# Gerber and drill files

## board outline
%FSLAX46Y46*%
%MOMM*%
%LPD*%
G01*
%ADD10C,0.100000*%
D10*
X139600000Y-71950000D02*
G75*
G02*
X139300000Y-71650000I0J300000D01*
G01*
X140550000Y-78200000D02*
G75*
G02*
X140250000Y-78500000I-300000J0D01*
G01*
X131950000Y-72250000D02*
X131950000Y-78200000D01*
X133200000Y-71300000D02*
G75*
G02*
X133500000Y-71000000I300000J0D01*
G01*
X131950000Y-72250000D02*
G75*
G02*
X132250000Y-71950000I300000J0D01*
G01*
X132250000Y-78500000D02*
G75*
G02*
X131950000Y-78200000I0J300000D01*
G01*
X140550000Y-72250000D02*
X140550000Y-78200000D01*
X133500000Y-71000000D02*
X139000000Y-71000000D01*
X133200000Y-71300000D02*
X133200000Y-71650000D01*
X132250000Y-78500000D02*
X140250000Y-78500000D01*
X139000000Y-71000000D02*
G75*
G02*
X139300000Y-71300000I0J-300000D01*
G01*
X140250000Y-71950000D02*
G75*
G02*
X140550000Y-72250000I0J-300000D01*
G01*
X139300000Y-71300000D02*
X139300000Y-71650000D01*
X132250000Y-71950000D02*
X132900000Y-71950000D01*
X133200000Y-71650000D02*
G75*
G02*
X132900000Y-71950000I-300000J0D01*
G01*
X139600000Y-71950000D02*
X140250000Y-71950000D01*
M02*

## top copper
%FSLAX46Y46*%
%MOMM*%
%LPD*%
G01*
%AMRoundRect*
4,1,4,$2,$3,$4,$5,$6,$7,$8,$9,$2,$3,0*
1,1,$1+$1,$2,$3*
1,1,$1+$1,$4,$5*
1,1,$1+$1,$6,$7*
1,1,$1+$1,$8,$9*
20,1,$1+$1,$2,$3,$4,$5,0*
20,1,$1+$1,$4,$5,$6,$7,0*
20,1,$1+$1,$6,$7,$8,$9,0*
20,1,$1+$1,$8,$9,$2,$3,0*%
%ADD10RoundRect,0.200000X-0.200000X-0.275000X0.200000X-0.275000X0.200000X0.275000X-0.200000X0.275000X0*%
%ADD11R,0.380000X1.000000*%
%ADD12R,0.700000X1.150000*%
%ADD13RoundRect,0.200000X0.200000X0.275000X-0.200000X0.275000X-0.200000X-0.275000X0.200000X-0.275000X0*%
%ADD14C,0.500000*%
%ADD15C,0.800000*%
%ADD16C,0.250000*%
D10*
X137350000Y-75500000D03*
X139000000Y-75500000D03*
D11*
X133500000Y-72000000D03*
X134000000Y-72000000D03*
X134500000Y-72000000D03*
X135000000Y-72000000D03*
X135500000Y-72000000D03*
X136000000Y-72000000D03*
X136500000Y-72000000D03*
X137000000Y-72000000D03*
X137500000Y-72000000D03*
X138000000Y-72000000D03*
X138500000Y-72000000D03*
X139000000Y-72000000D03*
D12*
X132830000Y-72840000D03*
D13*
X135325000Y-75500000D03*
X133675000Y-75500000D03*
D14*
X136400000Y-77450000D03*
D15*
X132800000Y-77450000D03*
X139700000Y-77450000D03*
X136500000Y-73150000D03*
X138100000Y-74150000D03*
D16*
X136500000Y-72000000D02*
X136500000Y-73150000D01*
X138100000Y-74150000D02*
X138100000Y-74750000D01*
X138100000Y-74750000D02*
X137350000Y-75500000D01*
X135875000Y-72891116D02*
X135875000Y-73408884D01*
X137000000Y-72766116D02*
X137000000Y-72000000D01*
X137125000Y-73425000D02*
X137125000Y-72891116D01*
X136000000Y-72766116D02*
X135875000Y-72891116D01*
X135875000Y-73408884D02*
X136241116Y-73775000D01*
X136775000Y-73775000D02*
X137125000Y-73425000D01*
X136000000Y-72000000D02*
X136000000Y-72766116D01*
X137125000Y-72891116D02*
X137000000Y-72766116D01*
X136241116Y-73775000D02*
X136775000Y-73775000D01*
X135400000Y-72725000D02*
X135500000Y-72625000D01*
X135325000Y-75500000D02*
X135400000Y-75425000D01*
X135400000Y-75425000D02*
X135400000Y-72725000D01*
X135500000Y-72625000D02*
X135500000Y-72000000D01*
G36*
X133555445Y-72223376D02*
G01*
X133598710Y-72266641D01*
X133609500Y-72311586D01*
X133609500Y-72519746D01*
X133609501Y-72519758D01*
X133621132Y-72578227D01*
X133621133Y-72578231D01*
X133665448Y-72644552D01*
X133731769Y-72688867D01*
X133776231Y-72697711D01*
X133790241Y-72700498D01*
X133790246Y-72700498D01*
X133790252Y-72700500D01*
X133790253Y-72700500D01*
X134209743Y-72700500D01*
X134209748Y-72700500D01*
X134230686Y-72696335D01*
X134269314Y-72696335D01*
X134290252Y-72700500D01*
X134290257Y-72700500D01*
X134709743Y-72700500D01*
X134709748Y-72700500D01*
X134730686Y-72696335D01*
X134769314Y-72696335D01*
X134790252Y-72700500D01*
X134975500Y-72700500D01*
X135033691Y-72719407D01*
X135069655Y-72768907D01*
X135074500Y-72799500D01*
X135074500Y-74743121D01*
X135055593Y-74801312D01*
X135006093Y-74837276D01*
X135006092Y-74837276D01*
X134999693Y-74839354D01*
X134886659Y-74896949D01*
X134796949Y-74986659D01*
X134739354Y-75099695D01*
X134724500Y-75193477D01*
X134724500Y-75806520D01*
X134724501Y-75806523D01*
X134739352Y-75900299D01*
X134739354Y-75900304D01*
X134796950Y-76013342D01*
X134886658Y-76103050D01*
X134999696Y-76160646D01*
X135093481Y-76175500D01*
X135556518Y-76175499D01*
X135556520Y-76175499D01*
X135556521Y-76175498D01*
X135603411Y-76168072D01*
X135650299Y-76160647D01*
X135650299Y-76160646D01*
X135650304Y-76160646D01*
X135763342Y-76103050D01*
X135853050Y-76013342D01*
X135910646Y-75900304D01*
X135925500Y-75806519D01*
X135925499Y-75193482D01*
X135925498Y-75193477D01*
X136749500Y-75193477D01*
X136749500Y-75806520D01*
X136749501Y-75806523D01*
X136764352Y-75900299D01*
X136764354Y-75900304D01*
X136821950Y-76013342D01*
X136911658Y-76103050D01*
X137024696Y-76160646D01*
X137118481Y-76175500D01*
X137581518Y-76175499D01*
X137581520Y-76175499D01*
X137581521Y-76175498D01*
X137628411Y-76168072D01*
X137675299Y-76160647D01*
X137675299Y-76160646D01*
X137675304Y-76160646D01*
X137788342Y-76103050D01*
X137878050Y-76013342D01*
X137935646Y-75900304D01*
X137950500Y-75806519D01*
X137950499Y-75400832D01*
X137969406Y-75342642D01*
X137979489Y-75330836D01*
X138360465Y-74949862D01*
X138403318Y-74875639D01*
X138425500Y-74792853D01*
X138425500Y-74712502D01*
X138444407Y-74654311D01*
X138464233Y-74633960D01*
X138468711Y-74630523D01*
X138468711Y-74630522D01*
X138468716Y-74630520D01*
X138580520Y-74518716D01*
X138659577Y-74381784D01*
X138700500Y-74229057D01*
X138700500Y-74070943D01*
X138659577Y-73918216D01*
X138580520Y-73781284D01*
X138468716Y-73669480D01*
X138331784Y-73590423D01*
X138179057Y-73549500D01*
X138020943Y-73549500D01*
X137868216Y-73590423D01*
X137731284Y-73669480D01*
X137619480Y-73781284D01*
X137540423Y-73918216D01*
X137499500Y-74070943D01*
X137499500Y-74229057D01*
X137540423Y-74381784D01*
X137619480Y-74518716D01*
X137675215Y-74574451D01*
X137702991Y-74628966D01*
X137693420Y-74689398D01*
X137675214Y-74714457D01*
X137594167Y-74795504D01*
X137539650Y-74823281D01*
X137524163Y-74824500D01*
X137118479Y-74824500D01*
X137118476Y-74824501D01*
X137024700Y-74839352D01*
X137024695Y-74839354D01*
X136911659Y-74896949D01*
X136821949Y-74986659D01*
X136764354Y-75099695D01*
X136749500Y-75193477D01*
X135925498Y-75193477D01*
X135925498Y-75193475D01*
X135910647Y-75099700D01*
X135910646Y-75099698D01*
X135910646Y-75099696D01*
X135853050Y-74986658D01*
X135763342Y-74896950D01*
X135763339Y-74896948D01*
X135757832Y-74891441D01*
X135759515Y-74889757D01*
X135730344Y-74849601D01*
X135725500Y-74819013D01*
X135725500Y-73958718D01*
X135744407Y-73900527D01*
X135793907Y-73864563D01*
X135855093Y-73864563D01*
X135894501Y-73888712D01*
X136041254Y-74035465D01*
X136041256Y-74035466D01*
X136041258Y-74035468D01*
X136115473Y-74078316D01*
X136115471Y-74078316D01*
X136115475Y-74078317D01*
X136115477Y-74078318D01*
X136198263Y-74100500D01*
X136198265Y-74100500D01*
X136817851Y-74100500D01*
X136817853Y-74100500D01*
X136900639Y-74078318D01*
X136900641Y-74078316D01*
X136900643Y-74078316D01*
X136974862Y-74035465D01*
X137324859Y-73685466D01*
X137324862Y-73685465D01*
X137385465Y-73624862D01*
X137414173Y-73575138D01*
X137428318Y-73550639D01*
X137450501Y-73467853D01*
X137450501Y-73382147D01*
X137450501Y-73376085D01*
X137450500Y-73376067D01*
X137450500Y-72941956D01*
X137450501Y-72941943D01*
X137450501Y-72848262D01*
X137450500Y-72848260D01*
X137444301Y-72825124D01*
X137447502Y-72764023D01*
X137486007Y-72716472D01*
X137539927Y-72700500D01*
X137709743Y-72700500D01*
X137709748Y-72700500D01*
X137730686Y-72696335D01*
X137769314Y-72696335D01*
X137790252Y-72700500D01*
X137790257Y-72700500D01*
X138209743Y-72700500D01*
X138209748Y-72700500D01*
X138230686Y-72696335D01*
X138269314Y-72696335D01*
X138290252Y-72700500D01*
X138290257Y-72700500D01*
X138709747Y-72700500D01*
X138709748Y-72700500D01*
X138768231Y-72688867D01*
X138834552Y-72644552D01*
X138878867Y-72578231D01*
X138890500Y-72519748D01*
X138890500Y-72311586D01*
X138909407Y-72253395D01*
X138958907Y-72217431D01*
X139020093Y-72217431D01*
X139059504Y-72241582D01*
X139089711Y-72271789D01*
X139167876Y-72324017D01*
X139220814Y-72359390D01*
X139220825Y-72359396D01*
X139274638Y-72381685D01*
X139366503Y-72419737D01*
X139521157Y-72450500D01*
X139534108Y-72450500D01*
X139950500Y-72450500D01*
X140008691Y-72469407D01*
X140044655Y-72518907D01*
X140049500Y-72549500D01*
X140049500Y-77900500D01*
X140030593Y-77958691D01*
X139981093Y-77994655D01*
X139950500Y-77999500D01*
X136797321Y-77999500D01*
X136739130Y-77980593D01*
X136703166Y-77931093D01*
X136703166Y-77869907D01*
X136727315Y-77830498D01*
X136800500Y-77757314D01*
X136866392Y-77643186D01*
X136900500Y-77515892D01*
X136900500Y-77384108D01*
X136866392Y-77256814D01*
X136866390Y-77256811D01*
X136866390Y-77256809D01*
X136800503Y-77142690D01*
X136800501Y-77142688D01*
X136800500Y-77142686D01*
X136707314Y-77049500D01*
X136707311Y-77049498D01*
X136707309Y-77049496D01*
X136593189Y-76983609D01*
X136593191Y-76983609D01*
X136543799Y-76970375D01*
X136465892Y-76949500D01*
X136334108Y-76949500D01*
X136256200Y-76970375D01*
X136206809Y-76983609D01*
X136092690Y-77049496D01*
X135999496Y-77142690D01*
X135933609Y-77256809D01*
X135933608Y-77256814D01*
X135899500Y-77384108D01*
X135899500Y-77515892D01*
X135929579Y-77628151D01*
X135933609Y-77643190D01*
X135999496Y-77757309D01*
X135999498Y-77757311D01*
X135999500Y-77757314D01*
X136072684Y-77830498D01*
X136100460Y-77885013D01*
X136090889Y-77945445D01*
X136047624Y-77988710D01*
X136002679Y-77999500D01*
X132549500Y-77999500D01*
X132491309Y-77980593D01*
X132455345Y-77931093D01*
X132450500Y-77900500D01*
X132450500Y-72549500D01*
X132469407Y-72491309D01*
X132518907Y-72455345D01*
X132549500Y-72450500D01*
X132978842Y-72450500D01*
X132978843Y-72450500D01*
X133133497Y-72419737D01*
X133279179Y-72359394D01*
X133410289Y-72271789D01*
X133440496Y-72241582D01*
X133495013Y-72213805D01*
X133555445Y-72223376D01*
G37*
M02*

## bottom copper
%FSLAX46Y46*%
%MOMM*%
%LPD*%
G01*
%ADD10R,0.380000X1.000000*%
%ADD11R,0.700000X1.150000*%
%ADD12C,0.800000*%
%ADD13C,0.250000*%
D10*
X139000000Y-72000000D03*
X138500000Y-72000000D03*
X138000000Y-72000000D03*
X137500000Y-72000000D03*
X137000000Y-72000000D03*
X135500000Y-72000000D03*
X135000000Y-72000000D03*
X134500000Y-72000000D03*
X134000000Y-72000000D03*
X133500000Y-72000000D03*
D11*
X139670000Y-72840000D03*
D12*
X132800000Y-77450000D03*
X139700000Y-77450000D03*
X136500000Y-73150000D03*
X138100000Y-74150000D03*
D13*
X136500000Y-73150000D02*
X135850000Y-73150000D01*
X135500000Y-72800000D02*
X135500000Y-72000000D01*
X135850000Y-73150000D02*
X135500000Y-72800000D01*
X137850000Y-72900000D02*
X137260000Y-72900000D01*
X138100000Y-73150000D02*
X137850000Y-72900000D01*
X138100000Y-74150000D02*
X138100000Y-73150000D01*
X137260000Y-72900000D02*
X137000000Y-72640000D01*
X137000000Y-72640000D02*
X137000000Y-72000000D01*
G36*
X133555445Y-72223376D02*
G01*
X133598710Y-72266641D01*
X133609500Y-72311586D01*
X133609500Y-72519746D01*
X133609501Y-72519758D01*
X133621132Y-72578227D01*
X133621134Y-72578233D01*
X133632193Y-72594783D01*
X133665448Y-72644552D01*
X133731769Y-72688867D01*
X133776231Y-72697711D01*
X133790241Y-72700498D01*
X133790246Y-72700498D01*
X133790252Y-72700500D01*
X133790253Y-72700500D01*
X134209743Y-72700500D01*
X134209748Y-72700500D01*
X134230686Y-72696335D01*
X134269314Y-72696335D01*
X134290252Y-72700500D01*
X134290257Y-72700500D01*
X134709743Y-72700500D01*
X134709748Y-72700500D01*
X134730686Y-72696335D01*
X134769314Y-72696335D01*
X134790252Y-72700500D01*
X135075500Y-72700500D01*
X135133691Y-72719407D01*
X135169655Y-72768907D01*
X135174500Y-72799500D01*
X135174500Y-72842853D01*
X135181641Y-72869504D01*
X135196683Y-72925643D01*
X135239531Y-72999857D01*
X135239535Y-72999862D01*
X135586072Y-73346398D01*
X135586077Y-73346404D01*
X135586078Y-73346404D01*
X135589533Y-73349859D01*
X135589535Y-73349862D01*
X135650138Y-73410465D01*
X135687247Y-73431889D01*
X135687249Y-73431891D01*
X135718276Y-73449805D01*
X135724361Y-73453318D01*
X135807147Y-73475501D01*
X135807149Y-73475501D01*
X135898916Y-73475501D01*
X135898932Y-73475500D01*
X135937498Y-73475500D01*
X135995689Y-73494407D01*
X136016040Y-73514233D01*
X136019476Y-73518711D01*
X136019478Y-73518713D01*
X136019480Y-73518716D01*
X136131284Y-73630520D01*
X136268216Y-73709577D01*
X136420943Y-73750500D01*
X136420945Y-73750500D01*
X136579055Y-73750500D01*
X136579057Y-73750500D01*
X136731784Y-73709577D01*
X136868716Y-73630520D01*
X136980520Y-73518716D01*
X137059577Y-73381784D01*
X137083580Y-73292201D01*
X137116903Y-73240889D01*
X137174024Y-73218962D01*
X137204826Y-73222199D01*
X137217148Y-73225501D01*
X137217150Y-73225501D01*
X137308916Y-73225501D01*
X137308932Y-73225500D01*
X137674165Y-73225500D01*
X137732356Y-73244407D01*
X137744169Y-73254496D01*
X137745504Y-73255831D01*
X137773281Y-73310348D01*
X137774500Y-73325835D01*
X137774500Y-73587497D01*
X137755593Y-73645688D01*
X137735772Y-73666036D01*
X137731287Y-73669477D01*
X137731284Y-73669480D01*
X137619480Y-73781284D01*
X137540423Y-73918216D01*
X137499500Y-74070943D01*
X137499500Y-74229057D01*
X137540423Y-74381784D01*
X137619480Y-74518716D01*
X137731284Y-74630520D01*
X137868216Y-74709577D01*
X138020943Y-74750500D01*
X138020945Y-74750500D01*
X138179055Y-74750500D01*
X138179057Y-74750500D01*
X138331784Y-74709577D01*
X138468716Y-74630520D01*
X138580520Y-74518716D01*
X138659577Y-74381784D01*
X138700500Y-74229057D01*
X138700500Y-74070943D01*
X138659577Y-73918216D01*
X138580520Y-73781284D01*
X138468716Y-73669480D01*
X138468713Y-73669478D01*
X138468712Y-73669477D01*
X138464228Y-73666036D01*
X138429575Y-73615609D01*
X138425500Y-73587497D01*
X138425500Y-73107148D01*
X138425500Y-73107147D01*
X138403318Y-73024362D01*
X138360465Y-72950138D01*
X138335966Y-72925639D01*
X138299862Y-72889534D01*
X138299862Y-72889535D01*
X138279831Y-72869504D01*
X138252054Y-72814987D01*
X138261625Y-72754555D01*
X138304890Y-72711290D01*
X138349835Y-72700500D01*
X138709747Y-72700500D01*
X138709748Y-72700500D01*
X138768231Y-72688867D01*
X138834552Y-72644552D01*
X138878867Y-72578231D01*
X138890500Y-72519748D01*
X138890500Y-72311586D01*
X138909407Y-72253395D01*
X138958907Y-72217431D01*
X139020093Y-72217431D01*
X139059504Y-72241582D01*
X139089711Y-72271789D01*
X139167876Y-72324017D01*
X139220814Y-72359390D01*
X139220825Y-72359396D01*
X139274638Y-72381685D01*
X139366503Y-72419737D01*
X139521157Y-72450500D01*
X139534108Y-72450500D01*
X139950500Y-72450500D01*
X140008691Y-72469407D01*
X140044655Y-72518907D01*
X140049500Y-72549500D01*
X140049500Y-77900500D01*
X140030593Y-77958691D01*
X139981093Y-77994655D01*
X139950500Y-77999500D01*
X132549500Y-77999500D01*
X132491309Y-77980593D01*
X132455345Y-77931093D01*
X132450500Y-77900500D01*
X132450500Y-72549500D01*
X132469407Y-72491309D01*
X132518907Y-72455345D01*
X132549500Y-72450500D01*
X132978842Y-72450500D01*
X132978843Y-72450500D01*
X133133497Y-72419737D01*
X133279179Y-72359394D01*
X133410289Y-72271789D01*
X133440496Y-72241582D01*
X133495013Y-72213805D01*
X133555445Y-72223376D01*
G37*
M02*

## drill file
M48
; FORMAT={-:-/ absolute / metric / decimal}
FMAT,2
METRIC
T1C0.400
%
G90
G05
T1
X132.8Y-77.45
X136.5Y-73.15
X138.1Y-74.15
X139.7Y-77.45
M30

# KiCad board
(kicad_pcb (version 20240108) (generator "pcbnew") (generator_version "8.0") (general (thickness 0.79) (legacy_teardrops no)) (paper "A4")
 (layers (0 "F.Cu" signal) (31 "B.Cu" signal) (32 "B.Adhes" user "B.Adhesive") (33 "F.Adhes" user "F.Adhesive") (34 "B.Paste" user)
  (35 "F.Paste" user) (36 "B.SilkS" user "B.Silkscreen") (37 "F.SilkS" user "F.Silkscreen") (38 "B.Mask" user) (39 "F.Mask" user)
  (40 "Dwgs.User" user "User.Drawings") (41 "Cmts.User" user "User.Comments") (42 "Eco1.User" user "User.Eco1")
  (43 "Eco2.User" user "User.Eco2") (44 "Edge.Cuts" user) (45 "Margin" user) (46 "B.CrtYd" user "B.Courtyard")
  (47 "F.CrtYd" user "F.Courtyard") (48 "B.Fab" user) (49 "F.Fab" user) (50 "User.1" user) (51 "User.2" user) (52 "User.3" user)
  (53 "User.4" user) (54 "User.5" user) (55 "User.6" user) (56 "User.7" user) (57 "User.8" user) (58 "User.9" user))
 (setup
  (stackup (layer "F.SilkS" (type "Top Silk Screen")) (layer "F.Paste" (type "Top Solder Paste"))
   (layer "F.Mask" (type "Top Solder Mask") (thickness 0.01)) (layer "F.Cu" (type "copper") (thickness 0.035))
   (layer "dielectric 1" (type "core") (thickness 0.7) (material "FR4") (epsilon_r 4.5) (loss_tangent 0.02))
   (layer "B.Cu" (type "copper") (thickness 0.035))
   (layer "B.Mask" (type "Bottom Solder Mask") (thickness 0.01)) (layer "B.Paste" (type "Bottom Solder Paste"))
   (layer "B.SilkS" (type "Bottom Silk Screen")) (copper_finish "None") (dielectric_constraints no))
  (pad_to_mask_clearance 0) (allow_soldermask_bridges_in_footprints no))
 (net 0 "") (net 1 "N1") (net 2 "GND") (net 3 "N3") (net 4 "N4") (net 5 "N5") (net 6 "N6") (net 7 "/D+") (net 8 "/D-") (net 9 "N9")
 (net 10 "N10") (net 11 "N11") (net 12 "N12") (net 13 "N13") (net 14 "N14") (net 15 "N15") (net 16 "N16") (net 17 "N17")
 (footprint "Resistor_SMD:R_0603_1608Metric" (layer "F.Cu") (at 138.175 75.5)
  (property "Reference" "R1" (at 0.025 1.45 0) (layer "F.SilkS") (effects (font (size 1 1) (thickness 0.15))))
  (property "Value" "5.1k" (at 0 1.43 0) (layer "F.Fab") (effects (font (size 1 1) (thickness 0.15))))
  (pad "1" smd roundrect (at -0.825 0) (size 0.8 0.95) (layers "F.Cu" "F.Paste" "F.Mask") (roundrect_rratio 0.25) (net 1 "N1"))
  (pad "2" smd roundrect (at 0.825 0) (size 0.8 0.95) (layers "F.Cu" "F.Paste" "F.Mask") (roundrect_rratio 0.25) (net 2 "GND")))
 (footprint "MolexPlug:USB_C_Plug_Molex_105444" (layer "F.Cu") (at 136.25 71.96)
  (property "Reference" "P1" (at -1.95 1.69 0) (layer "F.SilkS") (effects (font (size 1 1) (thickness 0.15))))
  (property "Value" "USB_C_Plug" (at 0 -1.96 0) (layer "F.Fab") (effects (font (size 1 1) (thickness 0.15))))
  (pad "A1" smd rect (at -2.75 0.04) (size 0.38 1) (layers "F.Cu" "F.Paste" "F.Mask") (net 2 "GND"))
  (pad "A2" smd rect (at -2.25 0.04) (size 0.38 1) (layers "F.Cu" "F.Paste" "F.Mask") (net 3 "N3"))
  (pad "A3" smd rect (at -1.75 0.04) (size 0.38 1) (layers "F.Cu" "F.Paste" "F.Mask") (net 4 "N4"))
  (pad "A4" smd rect (at -1.25 0.04) (size 0.38 1) (layers "F.Cu" "F.Paste" "F.Mask") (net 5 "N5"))
  (pad "A5" smd rect (at -0.75 0.04) (size 0.38 1) (layers "F.Cu" "F.Paste" "F.Mask") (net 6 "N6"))
  (pad "A6" smd rect (at -0.25 0.04) (size 0.38 1) (layers "F.Cu" "F.Paste" "F.Mask") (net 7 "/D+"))
  (pad "A7" smd rect (at 0.25 0.04) (size 0.38 1) (layers "F.Cu" "F.Paste" "F.Mask") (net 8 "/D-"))
  (pad "A8" smd rect (at 0.75 0.04) (size 0.38 1) (layers "F.Cu" "F.Paste" "F.Mask") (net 7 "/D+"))
  (pad "A9" smd rect (at 1.25 0.04) (size 0.38 1) (layers "F.Cu" "F.Paste" "F.Mask") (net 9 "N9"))
  (pad "A10" smd rect (at 1.75 0.04) (size 0.38 1) (layers "F.Cu" "F.Paste" "F.Mask") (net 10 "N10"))
  (pad "A11" smd rect (at 2.25 0.04) (size 0.38 1) (layers "F.Cu" "F.Paste" "F.Mask") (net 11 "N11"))
  (pad "A12" smd rect (at 2.75 0.04) (size 0.38 1) (layers "F.Cu" "F.Paste" "F.Mask") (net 2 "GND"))
  (pad "B1" smd rect (at 2.75 0.04) (size 0.38 1) (layers "B.Cu" "B.Paste" "B.Mask") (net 2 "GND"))
  (pad "B2" smd rect (at 2.25 0.04) (size 0.38 1) (layers "B.Cu" "B.Paste" "B.Mask") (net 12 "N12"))
  (pad "B3" smd rect (at 1.75 0.04) (size 0.38 1) (layers "B.Cu" "B.Paste" "B.Mask") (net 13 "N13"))
  (pad "B4" smd rect (at 1.25 0.04) (size 0.38 1) (layers "B.Cu" "B.Paste" "B.Mask") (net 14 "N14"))
  (pad "B5" smd rect (at 0.75 0.04) (size 0.38 1) (layers "B.Cu" "B.Paste" "B.Mask") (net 1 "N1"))
  (pad "B8" smd rect (at -0.75 0.04) (size 0.38 1) (layers "B.Cu" "B.Paste" "B.Mask") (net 8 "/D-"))
  (pad "B9" smd rect (at -1.25 0.04) (size 0.38 1) (layers "B.Cu" "B.Paste" "B.Mask") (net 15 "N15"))
  (pad "B10" smd rect (at -1.75 0.04) (size 0.38 1) (layers "B.Cu" "B.Paste" "B.Mask") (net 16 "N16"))
  (pad "B11" smd rect (at -2.25 0.04) (size 0.38 1) (layers "B.Cu" "B.Paste" "B.Mask") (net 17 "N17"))
  (pad "B12" smd rect (at -2.75 0.04) (size 0.38 1) (layers "B.Cu" "B.Paste" "B.Mask") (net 2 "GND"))
  (pad "S1" smd rect (at -3.42 0.88) (size 0.7 1.15) (layers "F.Cu" "F.Paste" "F.Mask") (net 2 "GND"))
  (pad "S1" smd rect (at 3.42 0.88) (size 0.7 1.15) (layers "B.Cu" "B.Paste" "B.Mask") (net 2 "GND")))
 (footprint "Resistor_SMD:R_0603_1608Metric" (layer "F.Cu") (at 134.5 75.5 180)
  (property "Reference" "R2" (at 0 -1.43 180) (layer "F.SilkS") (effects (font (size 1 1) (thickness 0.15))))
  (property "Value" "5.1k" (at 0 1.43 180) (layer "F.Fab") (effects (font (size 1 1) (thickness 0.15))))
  (pad "1" smd roundrect (at -0.825 0 180) (size 0.8 0.95) (layers "F.Cu" "F.Paste" "F.Mask") (roundrect_rratio 0.25) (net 6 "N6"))
  (pad "2" smd roundrect (at 0.825 0 180) (size 0.8 0.95) (layers "F.Cu" "F.Paste" "F.Mask") (roundrect_rratio 0.25) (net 2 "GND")))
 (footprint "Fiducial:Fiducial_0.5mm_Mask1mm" (layer "F.Cu") (at 136.4 77.45)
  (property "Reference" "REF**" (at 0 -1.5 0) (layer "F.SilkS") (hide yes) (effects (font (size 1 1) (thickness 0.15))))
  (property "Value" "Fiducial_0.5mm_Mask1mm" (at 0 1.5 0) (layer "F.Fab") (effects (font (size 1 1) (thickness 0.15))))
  (pad "" smd circle (at 0 0) (size 0.5 0.5) (layers "F.Cu" "F.Mask") (solder_mask_margin 0.25) (clearance 0.25)))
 (gr_arc (start 139.6 71.95) (mid 139.387868 71.862132) (end 139.3 71.65) (stroke (width 0.1) (type default)) (layer "Edge.Cuts"))
 (gr_arc (start 140.55 78.2) (mid 140.462132 78.412132) (end 140.25 78.5) (stroke (width 0.1) (type default)) (layer "Edge.Cuts"))
 (gr_line (start 131.95 72.25) (end 131.95 78.2) (stroke (width 0.1) (type default)) (layer "Edge.Cuts"))
 (gr_arc (start 133.2 71.3) (mid 133.287868 71.087868) (end 133.5 71) (stroke (width 0.1) (type default)) (layer "Edge.Cuts"))
 (gr_arc (start 131.95 72.25) (mid 132.037868 72.037868) (end 132.25 71.95) (stroke (width 0.1) (type default)) (layer "Edge.Cuts"))
 (gr_arc (start 132.25 78.5) (mid 132.037868 78.412132) (end 131.95 78.2) (stroke (width 0.1) (type default)) (layer "Edge.Cuts"))
 (gr_line (start 140.55 72.25) (end 140.55 78.2) (stroke (width 0.1) (type default)) (layer "Edge.Cuts"))
 (gr_line (start 133.5 71) (end 139 71) (stroke (width 0.1) (type default)) (layer "Edge.Cuts"))
 (gr_line (start 133.2 71.3) (end 133.2 71.65) (stroke (width 0.1) (type default)) (layer "Edge.Cuts"))
 (gr_line (start 132.25 78.5) (end 140.25 78.5) (stroke (width 0.1) (type default)) (layer "Edge.Cuts"))
 (gr_arc (start 139 71) (mid 139.212132 71.087868) (end 139.3 71.3) (stroke (width 0.1) (type default)) (layer "Edge.Cuts"))
 (gr_arc (start 140.25 71.95) (mid 140.462132 72.037868) (end 140.55 72.25) (stroke (width 0.1) (type default)) (layer "Edge.Cuts"))
 (gr_line (start 139.3 71.3) (end 139.3 71.65) (stroke (width 0.1) (type default)) (layer "Edge.Cuts"))
 (gr_line (start 132.25 71.95) (end 132.9 71.95) (stroke (width 0.1) (type default)) (layer "Edge.Cuts"))
 (gr_arc (start 133.2 71.65) (mid 133.112132 71.862132) (end 132.9 71.95) (stroke (width 0.1) (type default)) (layer "Edge.Cuts"))
 (gr_line (start 139.6 71.95) (end 140.25 71.95) (stroke (width 0.1) (type default)) (layer "Edge.Cuts"))
 (via (at 132.8 77.45) (size 0.8) (drill 0.4) (layers "F.Cu" "B.Cu") (free yes) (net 2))
 (via (at 139.7 77.45) (size 0.8) (drill 0.4) (layers "F.Cu" "B.Cu") (free yes) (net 2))
 (segment (start 136.5 72) (end 136.5 73.15) (width 0.25) (layer "F.Cu") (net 8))
 (via (at 136.5 73.15) (size 0.8) (drill 0.4) (layers "F.Cu" "B.Cu") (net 8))
 (segment (start 136.5 73.15) (end 135.85 73.15) (width 0.25) (layer "B.Cu") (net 8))
 (segment (start 135.5 72.8) (end 135.5 72) (width 0.25) (layer "B.Cu") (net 8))
 (segment (start 135.85 73.15) (end 135.5 72.8) (width 0.25) (layer "B.Cu") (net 8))
 (segment (start 138.1 74.15) (end 138.1 74.75) (width 0.25) (layer "F.Cu") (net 1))
 (segment (start 138.1 74.75) (end 137.35 75.5) (width 0.25) (layer "F.Cu") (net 1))
 (via (at 138.1 74.15) (size 0.8) (drill 0.4) (layers "F.Cu" "B.Cu") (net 1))
 (segment (start 137.85 72.9) (end 137.26 72.9) (width 0.25) (layer "B.Cu") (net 1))
 (segment (start 138.1 73.15) (end 137.85 72.9) (width 0.25) (layer "B.Cu") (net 1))
 (segment (start 138.1 74.15) (end 138.1 73.15) (width 0.25) (layer "B.Cu") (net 1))
 (segment (start 137.26 72.9) (end 137 72.64) (width 0.25) (layer "B.Cu") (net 1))
 (segment (start 137 72.64) (end 137 72) (width 0.25) (layer "B.Cu") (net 1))
 (segment (start 135.875 72.891116) (end 135.875 73.408884) (width 0.25) (layer "F.Cu") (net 7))
 (segment (start 137 72.766116) (end 137 72) (width 0.25) (layer "F.Cu") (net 7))
 (segment (start 137.125 73.425) (end 137.125 72.891116) (width 0.25) (layer "F.Cu") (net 7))
 (segment (start 136 72.766116) (end 135.875 72.891116) (width 0.25) (layer "F.Cu") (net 7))
 (segment (start 135.875 73.408884) (end 136.241116 73.775) (width 0.25) (layer "F.Cu") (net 7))
 (segment (start 136.775 73.775) (end 137.125 73.425) (width 0.25) (layer "F.Cu") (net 7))
 (segment (start 136 72) (end 136 72.766116) (width 0.25) (layer "F.Cu") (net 7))
 (segment (start 137.125 72.891116) (end 137 72.766116) (width 0.25) (layer "F.Cu") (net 7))
 (segment (start 136.241116 73.775) (end 136.775 73.775) (width 0.25) (layer "F.Cu") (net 7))
 (segment (start 135.4 72.725) (end 135.5 72.625) (width 0.25) (layer "F.Cu") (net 6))
 (segment (start 135.325 75.5) (end 135.4 75.425) (width 0.25) (layer "F.Cu") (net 6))
 (segment (start 135.4 75.425) (end 135.4 72.725) (width 0.25) (layer "F.Cu") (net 6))
 (segment (start 135.5 72.625) (end 135.5 72) (width 0.25) (layer "F.Cu") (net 6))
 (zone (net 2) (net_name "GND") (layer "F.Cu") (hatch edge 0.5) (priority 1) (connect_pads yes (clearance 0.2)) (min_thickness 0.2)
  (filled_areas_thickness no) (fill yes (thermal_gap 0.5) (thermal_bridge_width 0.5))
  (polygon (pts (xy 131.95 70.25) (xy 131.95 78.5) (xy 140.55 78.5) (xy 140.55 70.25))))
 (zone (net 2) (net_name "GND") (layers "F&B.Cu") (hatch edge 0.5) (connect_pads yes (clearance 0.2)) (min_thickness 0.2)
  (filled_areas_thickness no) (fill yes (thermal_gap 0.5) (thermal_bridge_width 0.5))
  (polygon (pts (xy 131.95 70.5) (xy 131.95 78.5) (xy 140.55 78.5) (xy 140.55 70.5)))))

